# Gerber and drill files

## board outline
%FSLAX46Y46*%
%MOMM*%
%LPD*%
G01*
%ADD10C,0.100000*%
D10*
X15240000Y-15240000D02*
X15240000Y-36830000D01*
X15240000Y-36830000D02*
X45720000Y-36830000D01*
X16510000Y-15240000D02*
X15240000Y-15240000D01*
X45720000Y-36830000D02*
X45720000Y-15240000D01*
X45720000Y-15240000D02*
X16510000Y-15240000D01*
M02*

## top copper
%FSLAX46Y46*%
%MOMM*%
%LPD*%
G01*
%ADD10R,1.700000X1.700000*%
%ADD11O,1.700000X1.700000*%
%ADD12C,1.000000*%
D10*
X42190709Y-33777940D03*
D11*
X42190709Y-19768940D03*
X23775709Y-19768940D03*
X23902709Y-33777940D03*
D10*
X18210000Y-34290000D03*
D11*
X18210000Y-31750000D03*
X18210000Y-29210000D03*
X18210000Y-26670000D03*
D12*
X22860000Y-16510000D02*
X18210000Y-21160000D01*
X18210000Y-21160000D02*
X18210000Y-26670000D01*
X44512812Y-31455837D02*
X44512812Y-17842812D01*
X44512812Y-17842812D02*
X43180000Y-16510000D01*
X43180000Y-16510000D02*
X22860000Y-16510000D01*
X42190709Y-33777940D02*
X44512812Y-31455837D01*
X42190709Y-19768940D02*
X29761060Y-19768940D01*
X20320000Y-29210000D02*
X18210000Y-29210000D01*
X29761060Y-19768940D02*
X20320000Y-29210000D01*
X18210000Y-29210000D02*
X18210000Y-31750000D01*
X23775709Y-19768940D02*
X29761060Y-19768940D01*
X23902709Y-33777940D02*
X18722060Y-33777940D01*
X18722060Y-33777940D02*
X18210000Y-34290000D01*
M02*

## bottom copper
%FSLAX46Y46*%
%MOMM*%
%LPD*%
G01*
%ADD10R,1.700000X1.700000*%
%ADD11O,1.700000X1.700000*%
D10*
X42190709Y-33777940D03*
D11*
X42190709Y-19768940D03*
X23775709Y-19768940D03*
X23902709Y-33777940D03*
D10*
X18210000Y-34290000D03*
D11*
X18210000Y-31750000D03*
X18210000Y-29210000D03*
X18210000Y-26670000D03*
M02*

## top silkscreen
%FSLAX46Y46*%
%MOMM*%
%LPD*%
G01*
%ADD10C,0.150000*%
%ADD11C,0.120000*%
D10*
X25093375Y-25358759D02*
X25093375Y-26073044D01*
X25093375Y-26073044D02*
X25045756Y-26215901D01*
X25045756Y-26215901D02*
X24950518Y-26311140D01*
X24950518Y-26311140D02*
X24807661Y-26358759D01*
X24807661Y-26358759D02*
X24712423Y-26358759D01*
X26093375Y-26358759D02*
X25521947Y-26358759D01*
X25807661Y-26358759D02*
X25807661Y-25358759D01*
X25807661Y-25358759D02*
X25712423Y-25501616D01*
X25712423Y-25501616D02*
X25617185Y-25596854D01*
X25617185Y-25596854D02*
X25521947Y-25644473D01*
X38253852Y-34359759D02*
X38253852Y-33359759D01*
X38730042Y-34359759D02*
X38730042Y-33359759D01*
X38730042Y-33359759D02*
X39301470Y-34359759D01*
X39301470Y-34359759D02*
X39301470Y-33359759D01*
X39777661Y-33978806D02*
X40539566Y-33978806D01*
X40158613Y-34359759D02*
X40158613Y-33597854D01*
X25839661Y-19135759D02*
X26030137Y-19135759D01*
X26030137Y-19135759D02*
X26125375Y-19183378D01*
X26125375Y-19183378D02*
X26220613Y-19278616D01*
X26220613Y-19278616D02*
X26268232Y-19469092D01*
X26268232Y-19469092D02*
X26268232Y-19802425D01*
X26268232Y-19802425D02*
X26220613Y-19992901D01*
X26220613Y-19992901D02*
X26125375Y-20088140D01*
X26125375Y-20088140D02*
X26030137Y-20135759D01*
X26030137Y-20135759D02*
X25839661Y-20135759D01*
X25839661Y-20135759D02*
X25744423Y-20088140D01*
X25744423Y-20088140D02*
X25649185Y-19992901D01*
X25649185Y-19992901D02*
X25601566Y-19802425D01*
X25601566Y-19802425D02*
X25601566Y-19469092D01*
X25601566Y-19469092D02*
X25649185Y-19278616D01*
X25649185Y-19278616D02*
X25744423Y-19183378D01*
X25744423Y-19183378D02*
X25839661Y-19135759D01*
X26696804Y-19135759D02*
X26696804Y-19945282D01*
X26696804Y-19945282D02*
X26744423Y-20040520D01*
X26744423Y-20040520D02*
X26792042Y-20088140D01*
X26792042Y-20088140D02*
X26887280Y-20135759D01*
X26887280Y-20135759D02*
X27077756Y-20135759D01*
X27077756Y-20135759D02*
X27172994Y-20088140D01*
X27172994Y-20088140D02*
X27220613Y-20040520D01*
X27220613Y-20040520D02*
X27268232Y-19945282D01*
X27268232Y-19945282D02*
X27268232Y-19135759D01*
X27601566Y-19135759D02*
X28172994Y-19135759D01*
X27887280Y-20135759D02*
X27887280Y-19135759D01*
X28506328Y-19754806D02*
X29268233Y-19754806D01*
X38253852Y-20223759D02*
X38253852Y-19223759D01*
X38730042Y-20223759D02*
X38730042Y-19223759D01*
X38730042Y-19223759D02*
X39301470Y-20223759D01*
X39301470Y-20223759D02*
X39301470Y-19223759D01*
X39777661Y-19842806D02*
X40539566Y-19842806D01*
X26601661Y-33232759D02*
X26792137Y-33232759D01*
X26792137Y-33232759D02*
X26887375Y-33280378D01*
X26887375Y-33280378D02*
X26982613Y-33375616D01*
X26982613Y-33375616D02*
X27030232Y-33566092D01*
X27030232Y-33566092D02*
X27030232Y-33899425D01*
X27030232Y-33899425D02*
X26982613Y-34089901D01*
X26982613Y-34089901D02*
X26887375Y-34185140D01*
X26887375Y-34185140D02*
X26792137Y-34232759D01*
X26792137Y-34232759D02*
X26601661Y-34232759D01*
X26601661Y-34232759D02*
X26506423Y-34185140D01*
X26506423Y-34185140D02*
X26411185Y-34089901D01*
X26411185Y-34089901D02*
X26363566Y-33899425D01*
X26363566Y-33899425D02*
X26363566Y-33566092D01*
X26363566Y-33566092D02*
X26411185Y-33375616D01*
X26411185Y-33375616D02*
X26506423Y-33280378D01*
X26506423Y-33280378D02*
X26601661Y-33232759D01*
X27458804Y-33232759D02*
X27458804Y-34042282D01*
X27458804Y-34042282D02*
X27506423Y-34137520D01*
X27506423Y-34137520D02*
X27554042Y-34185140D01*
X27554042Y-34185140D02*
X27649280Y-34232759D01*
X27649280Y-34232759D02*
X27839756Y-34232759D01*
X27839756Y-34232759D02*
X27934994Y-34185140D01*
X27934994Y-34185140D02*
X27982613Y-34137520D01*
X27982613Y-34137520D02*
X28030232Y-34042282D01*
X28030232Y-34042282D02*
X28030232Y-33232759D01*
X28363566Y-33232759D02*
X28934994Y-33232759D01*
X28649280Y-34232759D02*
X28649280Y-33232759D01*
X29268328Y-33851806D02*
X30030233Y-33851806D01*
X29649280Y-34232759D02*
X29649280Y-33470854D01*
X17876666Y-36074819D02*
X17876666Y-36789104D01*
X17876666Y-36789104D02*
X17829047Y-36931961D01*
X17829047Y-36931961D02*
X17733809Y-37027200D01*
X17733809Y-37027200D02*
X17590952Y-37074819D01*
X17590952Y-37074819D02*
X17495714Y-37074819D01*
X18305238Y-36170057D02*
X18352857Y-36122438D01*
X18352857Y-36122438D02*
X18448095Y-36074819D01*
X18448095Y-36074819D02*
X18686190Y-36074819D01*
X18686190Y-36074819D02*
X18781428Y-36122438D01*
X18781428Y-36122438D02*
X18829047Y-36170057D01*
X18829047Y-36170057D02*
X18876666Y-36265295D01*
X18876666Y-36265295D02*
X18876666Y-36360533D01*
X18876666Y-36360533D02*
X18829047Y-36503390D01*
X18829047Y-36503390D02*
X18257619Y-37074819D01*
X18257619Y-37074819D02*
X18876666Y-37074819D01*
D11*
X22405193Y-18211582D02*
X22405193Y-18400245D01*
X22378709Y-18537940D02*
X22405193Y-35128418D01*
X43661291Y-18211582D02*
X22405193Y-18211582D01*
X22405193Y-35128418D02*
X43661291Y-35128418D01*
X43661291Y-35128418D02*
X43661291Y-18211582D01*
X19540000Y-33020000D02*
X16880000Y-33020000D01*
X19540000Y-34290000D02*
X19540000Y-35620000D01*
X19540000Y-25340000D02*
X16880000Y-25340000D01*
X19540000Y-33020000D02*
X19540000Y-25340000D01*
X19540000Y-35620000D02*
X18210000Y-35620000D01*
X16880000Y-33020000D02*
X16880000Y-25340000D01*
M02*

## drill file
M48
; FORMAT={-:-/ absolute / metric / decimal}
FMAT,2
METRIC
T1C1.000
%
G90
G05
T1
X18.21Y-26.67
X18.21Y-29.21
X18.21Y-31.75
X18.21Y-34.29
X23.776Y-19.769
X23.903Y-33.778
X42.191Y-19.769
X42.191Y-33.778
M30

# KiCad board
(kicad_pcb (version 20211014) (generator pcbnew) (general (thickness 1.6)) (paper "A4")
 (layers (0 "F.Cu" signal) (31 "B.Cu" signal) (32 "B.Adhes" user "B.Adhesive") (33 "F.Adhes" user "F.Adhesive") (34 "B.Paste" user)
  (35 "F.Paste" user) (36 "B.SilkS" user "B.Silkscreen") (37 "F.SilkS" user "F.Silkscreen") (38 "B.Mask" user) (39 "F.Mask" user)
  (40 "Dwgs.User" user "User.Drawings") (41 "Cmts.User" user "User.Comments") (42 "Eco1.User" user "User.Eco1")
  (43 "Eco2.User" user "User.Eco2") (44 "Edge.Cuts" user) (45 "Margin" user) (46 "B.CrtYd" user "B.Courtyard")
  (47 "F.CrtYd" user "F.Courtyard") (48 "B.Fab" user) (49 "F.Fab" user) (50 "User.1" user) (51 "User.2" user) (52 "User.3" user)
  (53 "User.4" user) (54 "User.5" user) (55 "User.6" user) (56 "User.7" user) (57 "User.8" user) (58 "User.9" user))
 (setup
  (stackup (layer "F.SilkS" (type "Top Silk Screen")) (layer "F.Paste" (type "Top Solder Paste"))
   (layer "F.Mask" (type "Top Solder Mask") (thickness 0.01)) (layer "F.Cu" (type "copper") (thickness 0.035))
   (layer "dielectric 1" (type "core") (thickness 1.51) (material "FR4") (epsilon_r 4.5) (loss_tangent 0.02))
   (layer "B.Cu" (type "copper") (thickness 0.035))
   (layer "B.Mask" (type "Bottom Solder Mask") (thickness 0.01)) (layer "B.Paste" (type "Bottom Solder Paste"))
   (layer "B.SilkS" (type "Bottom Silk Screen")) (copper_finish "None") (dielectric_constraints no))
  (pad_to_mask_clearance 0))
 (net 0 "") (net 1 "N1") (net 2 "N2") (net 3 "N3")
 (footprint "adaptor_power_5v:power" (layer "F.Cu") (at 23.775709 19.76894)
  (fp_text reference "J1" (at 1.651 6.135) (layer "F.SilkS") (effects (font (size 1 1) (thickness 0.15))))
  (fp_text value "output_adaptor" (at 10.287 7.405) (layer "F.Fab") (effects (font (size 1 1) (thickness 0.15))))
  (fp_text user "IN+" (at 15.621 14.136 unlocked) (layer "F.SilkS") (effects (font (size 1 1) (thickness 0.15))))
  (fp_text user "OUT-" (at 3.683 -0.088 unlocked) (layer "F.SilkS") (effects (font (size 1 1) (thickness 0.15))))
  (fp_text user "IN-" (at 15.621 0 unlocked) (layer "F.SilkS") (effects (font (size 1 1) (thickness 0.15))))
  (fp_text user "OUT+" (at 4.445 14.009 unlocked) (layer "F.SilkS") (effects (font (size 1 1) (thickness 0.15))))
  (fp_line (start -1.370516 -1.557358) (end -1.370516 -1.368695) (layer "F.SilkS") (width 0.12))
  (fp_line (start -1.397 -1.231) (end -1.370516 15.359478) (layer "F.SilkS") (width 0.12))
  (fp_line (start 19.885582 -1.557358) (end -1.370516 -1.557358) (layer "F.SilkS") (width 0.12))
  (fp_line (start -1.370516 15.359478) (end 19.885582 15.359478) (layer "F.SilkS") (width 0.12))
  (fp_line (start 19.885582 15.359478) (end 19.885582 -1.557358) (layer "F.SilkS") (width 0.12))
  (pad "1" thru_hole rect (at 18.415 14.009) (size 1.7 1.7) (drill 1) (layers *.Cu *.Mask) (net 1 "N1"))
  (pad "2" thru_hole oval (at 18.415 0) (size 1.7 1.7) (drill 1) (layers *.Cu *.Mask) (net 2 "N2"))
  (pad "3" thru_hole oval (at 0 0) (size 1.7 1.7) (drill 1) (layers *.Cu *.Mask) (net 2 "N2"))
  (pad "4" thru_hole oval (at 0.127 14.009) (size 1.7 1.7) (drill 1) (layers *.Cu *.Mask) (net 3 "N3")))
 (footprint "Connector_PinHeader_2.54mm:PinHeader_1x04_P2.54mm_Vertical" (layer "F.Cu") (at 18.21 34.29 180)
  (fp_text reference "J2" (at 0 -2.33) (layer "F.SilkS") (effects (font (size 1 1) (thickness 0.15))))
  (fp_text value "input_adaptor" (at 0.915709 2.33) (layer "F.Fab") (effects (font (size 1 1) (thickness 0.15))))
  (fp_line (start -1.33 1.27) (end 1.33 1.27) (layer "F.SilkS") (width 0.12))
  (fp_line (start -1.33 0) (end -1.33 -1.33) (layer "F.SilkS") (width 0.12))
  (fp_line (start -1.33 8.95) (end 1.33 8.95) (layer "F.SilkS") (width 0.12))
  (fp_line (start -1.33 1.27) (end -1.33 8.95) (layer "F.SilkS") (width 0.12))
  (fp_line (start -1.33 -1.33) (end 0 -1.33) (layer "F.SilkS") (width 0.12))
  (fp_line (start 1.33 1.27) (end 1.33 8.95) (layer "F.SilkS") (width 0.12))
  (pad "1" thru_hole rect (at 0 0 180) (size 1.7 1.7) (drill 1) (layers *.Cu *.Mask) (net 3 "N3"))
  (pad "2" thru_hole oval (at 0 2.54 180) (size 1.7 1.7) (drill 1) (layers *.Cu *.Mask) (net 2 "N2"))
  (pad "3" thru_hole oval (at 0 5.08 180) (size 1.7 1.7) (drill 1) (layers *.Cu *.Mask) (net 2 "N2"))
  (pad "4" thru_hole oval (at 0 7.62 180) (size 1.7 1.7) (drill 1) (layers *.Cu *.Mask) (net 1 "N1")))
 (gr_line (start 15.24 15.24) (end 15.24 36.83) (layer "Edge.Cuts") (width 0.1))
 (gr_line (start 15.24 36.83) (end 45.72 36.83) (layer "Edge.Cuts") (width 0.1))
 (gr_line (start 16.51 15.24) (end 15.24 15.24) (layer "Edge.Cuts") (width 0.1))
 (gr_line (start 45.72 36.83) (end 45.72 15.24) (layer "Edge.Cuts") (width 0.1))
 (gr_line (start 45.72 15.24) (end 16.51 15.24) (layer "Edge.Cuts") (width 0.1))
 (segment (start 22.86 16.51) (end 18.21 21.16) (width 1) (layer "F.Cu") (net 1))
 (segment (start 18.21 21.16) (end 18.21 26.67) (width 1) (layer "F.Cu") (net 1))
 (segment (start 44.512812 31.455837) (end 44.512812 17.842812) (width 1) (layer "F.Cu") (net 1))
 (segment (start 44.512812 17.842812) (end 43.18 16.51) (width 1) (layer "F.Cu") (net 1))
 (segment (start 43.18 16.51) (end 22.86 16.51) (width 1) (layer "F.Cu") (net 1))
 (segment (start 42.190709 33.77794) (end 44.512812 31.455837) (width 1) (layer "F.Cu") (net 1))
 (segment (start 42.190709 19.76894) (end 29.76106 19.76894) (width 1) (layer "F.Cu") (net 2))
 (segment (start 20.32 29.21) (end 18.21 29.21) (width 1) (layer "F.Cu") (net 2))
 (segment (start 29.76106 19.76894) (end 20.32 29.21) (width 1) (layer "F.Cu") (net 2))
 (segment (start 18.21 29.21) (end 18.21 31.75) (width 1) (layer "F.Cu") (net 2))
 (segment (start 23.775709 19.76894) (end 29.76106 19.76894) (width 1) (layer "F.Cu") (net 2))
 (segment (start 23.902709 33.77794) (end 18.72206 33.77794) (width 1) (layer "F.Cu") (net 3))
 (segment (start 18.72206 33.77794) (end 18.21 34.29) (width 1) (layer "F.Cu") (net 3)))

